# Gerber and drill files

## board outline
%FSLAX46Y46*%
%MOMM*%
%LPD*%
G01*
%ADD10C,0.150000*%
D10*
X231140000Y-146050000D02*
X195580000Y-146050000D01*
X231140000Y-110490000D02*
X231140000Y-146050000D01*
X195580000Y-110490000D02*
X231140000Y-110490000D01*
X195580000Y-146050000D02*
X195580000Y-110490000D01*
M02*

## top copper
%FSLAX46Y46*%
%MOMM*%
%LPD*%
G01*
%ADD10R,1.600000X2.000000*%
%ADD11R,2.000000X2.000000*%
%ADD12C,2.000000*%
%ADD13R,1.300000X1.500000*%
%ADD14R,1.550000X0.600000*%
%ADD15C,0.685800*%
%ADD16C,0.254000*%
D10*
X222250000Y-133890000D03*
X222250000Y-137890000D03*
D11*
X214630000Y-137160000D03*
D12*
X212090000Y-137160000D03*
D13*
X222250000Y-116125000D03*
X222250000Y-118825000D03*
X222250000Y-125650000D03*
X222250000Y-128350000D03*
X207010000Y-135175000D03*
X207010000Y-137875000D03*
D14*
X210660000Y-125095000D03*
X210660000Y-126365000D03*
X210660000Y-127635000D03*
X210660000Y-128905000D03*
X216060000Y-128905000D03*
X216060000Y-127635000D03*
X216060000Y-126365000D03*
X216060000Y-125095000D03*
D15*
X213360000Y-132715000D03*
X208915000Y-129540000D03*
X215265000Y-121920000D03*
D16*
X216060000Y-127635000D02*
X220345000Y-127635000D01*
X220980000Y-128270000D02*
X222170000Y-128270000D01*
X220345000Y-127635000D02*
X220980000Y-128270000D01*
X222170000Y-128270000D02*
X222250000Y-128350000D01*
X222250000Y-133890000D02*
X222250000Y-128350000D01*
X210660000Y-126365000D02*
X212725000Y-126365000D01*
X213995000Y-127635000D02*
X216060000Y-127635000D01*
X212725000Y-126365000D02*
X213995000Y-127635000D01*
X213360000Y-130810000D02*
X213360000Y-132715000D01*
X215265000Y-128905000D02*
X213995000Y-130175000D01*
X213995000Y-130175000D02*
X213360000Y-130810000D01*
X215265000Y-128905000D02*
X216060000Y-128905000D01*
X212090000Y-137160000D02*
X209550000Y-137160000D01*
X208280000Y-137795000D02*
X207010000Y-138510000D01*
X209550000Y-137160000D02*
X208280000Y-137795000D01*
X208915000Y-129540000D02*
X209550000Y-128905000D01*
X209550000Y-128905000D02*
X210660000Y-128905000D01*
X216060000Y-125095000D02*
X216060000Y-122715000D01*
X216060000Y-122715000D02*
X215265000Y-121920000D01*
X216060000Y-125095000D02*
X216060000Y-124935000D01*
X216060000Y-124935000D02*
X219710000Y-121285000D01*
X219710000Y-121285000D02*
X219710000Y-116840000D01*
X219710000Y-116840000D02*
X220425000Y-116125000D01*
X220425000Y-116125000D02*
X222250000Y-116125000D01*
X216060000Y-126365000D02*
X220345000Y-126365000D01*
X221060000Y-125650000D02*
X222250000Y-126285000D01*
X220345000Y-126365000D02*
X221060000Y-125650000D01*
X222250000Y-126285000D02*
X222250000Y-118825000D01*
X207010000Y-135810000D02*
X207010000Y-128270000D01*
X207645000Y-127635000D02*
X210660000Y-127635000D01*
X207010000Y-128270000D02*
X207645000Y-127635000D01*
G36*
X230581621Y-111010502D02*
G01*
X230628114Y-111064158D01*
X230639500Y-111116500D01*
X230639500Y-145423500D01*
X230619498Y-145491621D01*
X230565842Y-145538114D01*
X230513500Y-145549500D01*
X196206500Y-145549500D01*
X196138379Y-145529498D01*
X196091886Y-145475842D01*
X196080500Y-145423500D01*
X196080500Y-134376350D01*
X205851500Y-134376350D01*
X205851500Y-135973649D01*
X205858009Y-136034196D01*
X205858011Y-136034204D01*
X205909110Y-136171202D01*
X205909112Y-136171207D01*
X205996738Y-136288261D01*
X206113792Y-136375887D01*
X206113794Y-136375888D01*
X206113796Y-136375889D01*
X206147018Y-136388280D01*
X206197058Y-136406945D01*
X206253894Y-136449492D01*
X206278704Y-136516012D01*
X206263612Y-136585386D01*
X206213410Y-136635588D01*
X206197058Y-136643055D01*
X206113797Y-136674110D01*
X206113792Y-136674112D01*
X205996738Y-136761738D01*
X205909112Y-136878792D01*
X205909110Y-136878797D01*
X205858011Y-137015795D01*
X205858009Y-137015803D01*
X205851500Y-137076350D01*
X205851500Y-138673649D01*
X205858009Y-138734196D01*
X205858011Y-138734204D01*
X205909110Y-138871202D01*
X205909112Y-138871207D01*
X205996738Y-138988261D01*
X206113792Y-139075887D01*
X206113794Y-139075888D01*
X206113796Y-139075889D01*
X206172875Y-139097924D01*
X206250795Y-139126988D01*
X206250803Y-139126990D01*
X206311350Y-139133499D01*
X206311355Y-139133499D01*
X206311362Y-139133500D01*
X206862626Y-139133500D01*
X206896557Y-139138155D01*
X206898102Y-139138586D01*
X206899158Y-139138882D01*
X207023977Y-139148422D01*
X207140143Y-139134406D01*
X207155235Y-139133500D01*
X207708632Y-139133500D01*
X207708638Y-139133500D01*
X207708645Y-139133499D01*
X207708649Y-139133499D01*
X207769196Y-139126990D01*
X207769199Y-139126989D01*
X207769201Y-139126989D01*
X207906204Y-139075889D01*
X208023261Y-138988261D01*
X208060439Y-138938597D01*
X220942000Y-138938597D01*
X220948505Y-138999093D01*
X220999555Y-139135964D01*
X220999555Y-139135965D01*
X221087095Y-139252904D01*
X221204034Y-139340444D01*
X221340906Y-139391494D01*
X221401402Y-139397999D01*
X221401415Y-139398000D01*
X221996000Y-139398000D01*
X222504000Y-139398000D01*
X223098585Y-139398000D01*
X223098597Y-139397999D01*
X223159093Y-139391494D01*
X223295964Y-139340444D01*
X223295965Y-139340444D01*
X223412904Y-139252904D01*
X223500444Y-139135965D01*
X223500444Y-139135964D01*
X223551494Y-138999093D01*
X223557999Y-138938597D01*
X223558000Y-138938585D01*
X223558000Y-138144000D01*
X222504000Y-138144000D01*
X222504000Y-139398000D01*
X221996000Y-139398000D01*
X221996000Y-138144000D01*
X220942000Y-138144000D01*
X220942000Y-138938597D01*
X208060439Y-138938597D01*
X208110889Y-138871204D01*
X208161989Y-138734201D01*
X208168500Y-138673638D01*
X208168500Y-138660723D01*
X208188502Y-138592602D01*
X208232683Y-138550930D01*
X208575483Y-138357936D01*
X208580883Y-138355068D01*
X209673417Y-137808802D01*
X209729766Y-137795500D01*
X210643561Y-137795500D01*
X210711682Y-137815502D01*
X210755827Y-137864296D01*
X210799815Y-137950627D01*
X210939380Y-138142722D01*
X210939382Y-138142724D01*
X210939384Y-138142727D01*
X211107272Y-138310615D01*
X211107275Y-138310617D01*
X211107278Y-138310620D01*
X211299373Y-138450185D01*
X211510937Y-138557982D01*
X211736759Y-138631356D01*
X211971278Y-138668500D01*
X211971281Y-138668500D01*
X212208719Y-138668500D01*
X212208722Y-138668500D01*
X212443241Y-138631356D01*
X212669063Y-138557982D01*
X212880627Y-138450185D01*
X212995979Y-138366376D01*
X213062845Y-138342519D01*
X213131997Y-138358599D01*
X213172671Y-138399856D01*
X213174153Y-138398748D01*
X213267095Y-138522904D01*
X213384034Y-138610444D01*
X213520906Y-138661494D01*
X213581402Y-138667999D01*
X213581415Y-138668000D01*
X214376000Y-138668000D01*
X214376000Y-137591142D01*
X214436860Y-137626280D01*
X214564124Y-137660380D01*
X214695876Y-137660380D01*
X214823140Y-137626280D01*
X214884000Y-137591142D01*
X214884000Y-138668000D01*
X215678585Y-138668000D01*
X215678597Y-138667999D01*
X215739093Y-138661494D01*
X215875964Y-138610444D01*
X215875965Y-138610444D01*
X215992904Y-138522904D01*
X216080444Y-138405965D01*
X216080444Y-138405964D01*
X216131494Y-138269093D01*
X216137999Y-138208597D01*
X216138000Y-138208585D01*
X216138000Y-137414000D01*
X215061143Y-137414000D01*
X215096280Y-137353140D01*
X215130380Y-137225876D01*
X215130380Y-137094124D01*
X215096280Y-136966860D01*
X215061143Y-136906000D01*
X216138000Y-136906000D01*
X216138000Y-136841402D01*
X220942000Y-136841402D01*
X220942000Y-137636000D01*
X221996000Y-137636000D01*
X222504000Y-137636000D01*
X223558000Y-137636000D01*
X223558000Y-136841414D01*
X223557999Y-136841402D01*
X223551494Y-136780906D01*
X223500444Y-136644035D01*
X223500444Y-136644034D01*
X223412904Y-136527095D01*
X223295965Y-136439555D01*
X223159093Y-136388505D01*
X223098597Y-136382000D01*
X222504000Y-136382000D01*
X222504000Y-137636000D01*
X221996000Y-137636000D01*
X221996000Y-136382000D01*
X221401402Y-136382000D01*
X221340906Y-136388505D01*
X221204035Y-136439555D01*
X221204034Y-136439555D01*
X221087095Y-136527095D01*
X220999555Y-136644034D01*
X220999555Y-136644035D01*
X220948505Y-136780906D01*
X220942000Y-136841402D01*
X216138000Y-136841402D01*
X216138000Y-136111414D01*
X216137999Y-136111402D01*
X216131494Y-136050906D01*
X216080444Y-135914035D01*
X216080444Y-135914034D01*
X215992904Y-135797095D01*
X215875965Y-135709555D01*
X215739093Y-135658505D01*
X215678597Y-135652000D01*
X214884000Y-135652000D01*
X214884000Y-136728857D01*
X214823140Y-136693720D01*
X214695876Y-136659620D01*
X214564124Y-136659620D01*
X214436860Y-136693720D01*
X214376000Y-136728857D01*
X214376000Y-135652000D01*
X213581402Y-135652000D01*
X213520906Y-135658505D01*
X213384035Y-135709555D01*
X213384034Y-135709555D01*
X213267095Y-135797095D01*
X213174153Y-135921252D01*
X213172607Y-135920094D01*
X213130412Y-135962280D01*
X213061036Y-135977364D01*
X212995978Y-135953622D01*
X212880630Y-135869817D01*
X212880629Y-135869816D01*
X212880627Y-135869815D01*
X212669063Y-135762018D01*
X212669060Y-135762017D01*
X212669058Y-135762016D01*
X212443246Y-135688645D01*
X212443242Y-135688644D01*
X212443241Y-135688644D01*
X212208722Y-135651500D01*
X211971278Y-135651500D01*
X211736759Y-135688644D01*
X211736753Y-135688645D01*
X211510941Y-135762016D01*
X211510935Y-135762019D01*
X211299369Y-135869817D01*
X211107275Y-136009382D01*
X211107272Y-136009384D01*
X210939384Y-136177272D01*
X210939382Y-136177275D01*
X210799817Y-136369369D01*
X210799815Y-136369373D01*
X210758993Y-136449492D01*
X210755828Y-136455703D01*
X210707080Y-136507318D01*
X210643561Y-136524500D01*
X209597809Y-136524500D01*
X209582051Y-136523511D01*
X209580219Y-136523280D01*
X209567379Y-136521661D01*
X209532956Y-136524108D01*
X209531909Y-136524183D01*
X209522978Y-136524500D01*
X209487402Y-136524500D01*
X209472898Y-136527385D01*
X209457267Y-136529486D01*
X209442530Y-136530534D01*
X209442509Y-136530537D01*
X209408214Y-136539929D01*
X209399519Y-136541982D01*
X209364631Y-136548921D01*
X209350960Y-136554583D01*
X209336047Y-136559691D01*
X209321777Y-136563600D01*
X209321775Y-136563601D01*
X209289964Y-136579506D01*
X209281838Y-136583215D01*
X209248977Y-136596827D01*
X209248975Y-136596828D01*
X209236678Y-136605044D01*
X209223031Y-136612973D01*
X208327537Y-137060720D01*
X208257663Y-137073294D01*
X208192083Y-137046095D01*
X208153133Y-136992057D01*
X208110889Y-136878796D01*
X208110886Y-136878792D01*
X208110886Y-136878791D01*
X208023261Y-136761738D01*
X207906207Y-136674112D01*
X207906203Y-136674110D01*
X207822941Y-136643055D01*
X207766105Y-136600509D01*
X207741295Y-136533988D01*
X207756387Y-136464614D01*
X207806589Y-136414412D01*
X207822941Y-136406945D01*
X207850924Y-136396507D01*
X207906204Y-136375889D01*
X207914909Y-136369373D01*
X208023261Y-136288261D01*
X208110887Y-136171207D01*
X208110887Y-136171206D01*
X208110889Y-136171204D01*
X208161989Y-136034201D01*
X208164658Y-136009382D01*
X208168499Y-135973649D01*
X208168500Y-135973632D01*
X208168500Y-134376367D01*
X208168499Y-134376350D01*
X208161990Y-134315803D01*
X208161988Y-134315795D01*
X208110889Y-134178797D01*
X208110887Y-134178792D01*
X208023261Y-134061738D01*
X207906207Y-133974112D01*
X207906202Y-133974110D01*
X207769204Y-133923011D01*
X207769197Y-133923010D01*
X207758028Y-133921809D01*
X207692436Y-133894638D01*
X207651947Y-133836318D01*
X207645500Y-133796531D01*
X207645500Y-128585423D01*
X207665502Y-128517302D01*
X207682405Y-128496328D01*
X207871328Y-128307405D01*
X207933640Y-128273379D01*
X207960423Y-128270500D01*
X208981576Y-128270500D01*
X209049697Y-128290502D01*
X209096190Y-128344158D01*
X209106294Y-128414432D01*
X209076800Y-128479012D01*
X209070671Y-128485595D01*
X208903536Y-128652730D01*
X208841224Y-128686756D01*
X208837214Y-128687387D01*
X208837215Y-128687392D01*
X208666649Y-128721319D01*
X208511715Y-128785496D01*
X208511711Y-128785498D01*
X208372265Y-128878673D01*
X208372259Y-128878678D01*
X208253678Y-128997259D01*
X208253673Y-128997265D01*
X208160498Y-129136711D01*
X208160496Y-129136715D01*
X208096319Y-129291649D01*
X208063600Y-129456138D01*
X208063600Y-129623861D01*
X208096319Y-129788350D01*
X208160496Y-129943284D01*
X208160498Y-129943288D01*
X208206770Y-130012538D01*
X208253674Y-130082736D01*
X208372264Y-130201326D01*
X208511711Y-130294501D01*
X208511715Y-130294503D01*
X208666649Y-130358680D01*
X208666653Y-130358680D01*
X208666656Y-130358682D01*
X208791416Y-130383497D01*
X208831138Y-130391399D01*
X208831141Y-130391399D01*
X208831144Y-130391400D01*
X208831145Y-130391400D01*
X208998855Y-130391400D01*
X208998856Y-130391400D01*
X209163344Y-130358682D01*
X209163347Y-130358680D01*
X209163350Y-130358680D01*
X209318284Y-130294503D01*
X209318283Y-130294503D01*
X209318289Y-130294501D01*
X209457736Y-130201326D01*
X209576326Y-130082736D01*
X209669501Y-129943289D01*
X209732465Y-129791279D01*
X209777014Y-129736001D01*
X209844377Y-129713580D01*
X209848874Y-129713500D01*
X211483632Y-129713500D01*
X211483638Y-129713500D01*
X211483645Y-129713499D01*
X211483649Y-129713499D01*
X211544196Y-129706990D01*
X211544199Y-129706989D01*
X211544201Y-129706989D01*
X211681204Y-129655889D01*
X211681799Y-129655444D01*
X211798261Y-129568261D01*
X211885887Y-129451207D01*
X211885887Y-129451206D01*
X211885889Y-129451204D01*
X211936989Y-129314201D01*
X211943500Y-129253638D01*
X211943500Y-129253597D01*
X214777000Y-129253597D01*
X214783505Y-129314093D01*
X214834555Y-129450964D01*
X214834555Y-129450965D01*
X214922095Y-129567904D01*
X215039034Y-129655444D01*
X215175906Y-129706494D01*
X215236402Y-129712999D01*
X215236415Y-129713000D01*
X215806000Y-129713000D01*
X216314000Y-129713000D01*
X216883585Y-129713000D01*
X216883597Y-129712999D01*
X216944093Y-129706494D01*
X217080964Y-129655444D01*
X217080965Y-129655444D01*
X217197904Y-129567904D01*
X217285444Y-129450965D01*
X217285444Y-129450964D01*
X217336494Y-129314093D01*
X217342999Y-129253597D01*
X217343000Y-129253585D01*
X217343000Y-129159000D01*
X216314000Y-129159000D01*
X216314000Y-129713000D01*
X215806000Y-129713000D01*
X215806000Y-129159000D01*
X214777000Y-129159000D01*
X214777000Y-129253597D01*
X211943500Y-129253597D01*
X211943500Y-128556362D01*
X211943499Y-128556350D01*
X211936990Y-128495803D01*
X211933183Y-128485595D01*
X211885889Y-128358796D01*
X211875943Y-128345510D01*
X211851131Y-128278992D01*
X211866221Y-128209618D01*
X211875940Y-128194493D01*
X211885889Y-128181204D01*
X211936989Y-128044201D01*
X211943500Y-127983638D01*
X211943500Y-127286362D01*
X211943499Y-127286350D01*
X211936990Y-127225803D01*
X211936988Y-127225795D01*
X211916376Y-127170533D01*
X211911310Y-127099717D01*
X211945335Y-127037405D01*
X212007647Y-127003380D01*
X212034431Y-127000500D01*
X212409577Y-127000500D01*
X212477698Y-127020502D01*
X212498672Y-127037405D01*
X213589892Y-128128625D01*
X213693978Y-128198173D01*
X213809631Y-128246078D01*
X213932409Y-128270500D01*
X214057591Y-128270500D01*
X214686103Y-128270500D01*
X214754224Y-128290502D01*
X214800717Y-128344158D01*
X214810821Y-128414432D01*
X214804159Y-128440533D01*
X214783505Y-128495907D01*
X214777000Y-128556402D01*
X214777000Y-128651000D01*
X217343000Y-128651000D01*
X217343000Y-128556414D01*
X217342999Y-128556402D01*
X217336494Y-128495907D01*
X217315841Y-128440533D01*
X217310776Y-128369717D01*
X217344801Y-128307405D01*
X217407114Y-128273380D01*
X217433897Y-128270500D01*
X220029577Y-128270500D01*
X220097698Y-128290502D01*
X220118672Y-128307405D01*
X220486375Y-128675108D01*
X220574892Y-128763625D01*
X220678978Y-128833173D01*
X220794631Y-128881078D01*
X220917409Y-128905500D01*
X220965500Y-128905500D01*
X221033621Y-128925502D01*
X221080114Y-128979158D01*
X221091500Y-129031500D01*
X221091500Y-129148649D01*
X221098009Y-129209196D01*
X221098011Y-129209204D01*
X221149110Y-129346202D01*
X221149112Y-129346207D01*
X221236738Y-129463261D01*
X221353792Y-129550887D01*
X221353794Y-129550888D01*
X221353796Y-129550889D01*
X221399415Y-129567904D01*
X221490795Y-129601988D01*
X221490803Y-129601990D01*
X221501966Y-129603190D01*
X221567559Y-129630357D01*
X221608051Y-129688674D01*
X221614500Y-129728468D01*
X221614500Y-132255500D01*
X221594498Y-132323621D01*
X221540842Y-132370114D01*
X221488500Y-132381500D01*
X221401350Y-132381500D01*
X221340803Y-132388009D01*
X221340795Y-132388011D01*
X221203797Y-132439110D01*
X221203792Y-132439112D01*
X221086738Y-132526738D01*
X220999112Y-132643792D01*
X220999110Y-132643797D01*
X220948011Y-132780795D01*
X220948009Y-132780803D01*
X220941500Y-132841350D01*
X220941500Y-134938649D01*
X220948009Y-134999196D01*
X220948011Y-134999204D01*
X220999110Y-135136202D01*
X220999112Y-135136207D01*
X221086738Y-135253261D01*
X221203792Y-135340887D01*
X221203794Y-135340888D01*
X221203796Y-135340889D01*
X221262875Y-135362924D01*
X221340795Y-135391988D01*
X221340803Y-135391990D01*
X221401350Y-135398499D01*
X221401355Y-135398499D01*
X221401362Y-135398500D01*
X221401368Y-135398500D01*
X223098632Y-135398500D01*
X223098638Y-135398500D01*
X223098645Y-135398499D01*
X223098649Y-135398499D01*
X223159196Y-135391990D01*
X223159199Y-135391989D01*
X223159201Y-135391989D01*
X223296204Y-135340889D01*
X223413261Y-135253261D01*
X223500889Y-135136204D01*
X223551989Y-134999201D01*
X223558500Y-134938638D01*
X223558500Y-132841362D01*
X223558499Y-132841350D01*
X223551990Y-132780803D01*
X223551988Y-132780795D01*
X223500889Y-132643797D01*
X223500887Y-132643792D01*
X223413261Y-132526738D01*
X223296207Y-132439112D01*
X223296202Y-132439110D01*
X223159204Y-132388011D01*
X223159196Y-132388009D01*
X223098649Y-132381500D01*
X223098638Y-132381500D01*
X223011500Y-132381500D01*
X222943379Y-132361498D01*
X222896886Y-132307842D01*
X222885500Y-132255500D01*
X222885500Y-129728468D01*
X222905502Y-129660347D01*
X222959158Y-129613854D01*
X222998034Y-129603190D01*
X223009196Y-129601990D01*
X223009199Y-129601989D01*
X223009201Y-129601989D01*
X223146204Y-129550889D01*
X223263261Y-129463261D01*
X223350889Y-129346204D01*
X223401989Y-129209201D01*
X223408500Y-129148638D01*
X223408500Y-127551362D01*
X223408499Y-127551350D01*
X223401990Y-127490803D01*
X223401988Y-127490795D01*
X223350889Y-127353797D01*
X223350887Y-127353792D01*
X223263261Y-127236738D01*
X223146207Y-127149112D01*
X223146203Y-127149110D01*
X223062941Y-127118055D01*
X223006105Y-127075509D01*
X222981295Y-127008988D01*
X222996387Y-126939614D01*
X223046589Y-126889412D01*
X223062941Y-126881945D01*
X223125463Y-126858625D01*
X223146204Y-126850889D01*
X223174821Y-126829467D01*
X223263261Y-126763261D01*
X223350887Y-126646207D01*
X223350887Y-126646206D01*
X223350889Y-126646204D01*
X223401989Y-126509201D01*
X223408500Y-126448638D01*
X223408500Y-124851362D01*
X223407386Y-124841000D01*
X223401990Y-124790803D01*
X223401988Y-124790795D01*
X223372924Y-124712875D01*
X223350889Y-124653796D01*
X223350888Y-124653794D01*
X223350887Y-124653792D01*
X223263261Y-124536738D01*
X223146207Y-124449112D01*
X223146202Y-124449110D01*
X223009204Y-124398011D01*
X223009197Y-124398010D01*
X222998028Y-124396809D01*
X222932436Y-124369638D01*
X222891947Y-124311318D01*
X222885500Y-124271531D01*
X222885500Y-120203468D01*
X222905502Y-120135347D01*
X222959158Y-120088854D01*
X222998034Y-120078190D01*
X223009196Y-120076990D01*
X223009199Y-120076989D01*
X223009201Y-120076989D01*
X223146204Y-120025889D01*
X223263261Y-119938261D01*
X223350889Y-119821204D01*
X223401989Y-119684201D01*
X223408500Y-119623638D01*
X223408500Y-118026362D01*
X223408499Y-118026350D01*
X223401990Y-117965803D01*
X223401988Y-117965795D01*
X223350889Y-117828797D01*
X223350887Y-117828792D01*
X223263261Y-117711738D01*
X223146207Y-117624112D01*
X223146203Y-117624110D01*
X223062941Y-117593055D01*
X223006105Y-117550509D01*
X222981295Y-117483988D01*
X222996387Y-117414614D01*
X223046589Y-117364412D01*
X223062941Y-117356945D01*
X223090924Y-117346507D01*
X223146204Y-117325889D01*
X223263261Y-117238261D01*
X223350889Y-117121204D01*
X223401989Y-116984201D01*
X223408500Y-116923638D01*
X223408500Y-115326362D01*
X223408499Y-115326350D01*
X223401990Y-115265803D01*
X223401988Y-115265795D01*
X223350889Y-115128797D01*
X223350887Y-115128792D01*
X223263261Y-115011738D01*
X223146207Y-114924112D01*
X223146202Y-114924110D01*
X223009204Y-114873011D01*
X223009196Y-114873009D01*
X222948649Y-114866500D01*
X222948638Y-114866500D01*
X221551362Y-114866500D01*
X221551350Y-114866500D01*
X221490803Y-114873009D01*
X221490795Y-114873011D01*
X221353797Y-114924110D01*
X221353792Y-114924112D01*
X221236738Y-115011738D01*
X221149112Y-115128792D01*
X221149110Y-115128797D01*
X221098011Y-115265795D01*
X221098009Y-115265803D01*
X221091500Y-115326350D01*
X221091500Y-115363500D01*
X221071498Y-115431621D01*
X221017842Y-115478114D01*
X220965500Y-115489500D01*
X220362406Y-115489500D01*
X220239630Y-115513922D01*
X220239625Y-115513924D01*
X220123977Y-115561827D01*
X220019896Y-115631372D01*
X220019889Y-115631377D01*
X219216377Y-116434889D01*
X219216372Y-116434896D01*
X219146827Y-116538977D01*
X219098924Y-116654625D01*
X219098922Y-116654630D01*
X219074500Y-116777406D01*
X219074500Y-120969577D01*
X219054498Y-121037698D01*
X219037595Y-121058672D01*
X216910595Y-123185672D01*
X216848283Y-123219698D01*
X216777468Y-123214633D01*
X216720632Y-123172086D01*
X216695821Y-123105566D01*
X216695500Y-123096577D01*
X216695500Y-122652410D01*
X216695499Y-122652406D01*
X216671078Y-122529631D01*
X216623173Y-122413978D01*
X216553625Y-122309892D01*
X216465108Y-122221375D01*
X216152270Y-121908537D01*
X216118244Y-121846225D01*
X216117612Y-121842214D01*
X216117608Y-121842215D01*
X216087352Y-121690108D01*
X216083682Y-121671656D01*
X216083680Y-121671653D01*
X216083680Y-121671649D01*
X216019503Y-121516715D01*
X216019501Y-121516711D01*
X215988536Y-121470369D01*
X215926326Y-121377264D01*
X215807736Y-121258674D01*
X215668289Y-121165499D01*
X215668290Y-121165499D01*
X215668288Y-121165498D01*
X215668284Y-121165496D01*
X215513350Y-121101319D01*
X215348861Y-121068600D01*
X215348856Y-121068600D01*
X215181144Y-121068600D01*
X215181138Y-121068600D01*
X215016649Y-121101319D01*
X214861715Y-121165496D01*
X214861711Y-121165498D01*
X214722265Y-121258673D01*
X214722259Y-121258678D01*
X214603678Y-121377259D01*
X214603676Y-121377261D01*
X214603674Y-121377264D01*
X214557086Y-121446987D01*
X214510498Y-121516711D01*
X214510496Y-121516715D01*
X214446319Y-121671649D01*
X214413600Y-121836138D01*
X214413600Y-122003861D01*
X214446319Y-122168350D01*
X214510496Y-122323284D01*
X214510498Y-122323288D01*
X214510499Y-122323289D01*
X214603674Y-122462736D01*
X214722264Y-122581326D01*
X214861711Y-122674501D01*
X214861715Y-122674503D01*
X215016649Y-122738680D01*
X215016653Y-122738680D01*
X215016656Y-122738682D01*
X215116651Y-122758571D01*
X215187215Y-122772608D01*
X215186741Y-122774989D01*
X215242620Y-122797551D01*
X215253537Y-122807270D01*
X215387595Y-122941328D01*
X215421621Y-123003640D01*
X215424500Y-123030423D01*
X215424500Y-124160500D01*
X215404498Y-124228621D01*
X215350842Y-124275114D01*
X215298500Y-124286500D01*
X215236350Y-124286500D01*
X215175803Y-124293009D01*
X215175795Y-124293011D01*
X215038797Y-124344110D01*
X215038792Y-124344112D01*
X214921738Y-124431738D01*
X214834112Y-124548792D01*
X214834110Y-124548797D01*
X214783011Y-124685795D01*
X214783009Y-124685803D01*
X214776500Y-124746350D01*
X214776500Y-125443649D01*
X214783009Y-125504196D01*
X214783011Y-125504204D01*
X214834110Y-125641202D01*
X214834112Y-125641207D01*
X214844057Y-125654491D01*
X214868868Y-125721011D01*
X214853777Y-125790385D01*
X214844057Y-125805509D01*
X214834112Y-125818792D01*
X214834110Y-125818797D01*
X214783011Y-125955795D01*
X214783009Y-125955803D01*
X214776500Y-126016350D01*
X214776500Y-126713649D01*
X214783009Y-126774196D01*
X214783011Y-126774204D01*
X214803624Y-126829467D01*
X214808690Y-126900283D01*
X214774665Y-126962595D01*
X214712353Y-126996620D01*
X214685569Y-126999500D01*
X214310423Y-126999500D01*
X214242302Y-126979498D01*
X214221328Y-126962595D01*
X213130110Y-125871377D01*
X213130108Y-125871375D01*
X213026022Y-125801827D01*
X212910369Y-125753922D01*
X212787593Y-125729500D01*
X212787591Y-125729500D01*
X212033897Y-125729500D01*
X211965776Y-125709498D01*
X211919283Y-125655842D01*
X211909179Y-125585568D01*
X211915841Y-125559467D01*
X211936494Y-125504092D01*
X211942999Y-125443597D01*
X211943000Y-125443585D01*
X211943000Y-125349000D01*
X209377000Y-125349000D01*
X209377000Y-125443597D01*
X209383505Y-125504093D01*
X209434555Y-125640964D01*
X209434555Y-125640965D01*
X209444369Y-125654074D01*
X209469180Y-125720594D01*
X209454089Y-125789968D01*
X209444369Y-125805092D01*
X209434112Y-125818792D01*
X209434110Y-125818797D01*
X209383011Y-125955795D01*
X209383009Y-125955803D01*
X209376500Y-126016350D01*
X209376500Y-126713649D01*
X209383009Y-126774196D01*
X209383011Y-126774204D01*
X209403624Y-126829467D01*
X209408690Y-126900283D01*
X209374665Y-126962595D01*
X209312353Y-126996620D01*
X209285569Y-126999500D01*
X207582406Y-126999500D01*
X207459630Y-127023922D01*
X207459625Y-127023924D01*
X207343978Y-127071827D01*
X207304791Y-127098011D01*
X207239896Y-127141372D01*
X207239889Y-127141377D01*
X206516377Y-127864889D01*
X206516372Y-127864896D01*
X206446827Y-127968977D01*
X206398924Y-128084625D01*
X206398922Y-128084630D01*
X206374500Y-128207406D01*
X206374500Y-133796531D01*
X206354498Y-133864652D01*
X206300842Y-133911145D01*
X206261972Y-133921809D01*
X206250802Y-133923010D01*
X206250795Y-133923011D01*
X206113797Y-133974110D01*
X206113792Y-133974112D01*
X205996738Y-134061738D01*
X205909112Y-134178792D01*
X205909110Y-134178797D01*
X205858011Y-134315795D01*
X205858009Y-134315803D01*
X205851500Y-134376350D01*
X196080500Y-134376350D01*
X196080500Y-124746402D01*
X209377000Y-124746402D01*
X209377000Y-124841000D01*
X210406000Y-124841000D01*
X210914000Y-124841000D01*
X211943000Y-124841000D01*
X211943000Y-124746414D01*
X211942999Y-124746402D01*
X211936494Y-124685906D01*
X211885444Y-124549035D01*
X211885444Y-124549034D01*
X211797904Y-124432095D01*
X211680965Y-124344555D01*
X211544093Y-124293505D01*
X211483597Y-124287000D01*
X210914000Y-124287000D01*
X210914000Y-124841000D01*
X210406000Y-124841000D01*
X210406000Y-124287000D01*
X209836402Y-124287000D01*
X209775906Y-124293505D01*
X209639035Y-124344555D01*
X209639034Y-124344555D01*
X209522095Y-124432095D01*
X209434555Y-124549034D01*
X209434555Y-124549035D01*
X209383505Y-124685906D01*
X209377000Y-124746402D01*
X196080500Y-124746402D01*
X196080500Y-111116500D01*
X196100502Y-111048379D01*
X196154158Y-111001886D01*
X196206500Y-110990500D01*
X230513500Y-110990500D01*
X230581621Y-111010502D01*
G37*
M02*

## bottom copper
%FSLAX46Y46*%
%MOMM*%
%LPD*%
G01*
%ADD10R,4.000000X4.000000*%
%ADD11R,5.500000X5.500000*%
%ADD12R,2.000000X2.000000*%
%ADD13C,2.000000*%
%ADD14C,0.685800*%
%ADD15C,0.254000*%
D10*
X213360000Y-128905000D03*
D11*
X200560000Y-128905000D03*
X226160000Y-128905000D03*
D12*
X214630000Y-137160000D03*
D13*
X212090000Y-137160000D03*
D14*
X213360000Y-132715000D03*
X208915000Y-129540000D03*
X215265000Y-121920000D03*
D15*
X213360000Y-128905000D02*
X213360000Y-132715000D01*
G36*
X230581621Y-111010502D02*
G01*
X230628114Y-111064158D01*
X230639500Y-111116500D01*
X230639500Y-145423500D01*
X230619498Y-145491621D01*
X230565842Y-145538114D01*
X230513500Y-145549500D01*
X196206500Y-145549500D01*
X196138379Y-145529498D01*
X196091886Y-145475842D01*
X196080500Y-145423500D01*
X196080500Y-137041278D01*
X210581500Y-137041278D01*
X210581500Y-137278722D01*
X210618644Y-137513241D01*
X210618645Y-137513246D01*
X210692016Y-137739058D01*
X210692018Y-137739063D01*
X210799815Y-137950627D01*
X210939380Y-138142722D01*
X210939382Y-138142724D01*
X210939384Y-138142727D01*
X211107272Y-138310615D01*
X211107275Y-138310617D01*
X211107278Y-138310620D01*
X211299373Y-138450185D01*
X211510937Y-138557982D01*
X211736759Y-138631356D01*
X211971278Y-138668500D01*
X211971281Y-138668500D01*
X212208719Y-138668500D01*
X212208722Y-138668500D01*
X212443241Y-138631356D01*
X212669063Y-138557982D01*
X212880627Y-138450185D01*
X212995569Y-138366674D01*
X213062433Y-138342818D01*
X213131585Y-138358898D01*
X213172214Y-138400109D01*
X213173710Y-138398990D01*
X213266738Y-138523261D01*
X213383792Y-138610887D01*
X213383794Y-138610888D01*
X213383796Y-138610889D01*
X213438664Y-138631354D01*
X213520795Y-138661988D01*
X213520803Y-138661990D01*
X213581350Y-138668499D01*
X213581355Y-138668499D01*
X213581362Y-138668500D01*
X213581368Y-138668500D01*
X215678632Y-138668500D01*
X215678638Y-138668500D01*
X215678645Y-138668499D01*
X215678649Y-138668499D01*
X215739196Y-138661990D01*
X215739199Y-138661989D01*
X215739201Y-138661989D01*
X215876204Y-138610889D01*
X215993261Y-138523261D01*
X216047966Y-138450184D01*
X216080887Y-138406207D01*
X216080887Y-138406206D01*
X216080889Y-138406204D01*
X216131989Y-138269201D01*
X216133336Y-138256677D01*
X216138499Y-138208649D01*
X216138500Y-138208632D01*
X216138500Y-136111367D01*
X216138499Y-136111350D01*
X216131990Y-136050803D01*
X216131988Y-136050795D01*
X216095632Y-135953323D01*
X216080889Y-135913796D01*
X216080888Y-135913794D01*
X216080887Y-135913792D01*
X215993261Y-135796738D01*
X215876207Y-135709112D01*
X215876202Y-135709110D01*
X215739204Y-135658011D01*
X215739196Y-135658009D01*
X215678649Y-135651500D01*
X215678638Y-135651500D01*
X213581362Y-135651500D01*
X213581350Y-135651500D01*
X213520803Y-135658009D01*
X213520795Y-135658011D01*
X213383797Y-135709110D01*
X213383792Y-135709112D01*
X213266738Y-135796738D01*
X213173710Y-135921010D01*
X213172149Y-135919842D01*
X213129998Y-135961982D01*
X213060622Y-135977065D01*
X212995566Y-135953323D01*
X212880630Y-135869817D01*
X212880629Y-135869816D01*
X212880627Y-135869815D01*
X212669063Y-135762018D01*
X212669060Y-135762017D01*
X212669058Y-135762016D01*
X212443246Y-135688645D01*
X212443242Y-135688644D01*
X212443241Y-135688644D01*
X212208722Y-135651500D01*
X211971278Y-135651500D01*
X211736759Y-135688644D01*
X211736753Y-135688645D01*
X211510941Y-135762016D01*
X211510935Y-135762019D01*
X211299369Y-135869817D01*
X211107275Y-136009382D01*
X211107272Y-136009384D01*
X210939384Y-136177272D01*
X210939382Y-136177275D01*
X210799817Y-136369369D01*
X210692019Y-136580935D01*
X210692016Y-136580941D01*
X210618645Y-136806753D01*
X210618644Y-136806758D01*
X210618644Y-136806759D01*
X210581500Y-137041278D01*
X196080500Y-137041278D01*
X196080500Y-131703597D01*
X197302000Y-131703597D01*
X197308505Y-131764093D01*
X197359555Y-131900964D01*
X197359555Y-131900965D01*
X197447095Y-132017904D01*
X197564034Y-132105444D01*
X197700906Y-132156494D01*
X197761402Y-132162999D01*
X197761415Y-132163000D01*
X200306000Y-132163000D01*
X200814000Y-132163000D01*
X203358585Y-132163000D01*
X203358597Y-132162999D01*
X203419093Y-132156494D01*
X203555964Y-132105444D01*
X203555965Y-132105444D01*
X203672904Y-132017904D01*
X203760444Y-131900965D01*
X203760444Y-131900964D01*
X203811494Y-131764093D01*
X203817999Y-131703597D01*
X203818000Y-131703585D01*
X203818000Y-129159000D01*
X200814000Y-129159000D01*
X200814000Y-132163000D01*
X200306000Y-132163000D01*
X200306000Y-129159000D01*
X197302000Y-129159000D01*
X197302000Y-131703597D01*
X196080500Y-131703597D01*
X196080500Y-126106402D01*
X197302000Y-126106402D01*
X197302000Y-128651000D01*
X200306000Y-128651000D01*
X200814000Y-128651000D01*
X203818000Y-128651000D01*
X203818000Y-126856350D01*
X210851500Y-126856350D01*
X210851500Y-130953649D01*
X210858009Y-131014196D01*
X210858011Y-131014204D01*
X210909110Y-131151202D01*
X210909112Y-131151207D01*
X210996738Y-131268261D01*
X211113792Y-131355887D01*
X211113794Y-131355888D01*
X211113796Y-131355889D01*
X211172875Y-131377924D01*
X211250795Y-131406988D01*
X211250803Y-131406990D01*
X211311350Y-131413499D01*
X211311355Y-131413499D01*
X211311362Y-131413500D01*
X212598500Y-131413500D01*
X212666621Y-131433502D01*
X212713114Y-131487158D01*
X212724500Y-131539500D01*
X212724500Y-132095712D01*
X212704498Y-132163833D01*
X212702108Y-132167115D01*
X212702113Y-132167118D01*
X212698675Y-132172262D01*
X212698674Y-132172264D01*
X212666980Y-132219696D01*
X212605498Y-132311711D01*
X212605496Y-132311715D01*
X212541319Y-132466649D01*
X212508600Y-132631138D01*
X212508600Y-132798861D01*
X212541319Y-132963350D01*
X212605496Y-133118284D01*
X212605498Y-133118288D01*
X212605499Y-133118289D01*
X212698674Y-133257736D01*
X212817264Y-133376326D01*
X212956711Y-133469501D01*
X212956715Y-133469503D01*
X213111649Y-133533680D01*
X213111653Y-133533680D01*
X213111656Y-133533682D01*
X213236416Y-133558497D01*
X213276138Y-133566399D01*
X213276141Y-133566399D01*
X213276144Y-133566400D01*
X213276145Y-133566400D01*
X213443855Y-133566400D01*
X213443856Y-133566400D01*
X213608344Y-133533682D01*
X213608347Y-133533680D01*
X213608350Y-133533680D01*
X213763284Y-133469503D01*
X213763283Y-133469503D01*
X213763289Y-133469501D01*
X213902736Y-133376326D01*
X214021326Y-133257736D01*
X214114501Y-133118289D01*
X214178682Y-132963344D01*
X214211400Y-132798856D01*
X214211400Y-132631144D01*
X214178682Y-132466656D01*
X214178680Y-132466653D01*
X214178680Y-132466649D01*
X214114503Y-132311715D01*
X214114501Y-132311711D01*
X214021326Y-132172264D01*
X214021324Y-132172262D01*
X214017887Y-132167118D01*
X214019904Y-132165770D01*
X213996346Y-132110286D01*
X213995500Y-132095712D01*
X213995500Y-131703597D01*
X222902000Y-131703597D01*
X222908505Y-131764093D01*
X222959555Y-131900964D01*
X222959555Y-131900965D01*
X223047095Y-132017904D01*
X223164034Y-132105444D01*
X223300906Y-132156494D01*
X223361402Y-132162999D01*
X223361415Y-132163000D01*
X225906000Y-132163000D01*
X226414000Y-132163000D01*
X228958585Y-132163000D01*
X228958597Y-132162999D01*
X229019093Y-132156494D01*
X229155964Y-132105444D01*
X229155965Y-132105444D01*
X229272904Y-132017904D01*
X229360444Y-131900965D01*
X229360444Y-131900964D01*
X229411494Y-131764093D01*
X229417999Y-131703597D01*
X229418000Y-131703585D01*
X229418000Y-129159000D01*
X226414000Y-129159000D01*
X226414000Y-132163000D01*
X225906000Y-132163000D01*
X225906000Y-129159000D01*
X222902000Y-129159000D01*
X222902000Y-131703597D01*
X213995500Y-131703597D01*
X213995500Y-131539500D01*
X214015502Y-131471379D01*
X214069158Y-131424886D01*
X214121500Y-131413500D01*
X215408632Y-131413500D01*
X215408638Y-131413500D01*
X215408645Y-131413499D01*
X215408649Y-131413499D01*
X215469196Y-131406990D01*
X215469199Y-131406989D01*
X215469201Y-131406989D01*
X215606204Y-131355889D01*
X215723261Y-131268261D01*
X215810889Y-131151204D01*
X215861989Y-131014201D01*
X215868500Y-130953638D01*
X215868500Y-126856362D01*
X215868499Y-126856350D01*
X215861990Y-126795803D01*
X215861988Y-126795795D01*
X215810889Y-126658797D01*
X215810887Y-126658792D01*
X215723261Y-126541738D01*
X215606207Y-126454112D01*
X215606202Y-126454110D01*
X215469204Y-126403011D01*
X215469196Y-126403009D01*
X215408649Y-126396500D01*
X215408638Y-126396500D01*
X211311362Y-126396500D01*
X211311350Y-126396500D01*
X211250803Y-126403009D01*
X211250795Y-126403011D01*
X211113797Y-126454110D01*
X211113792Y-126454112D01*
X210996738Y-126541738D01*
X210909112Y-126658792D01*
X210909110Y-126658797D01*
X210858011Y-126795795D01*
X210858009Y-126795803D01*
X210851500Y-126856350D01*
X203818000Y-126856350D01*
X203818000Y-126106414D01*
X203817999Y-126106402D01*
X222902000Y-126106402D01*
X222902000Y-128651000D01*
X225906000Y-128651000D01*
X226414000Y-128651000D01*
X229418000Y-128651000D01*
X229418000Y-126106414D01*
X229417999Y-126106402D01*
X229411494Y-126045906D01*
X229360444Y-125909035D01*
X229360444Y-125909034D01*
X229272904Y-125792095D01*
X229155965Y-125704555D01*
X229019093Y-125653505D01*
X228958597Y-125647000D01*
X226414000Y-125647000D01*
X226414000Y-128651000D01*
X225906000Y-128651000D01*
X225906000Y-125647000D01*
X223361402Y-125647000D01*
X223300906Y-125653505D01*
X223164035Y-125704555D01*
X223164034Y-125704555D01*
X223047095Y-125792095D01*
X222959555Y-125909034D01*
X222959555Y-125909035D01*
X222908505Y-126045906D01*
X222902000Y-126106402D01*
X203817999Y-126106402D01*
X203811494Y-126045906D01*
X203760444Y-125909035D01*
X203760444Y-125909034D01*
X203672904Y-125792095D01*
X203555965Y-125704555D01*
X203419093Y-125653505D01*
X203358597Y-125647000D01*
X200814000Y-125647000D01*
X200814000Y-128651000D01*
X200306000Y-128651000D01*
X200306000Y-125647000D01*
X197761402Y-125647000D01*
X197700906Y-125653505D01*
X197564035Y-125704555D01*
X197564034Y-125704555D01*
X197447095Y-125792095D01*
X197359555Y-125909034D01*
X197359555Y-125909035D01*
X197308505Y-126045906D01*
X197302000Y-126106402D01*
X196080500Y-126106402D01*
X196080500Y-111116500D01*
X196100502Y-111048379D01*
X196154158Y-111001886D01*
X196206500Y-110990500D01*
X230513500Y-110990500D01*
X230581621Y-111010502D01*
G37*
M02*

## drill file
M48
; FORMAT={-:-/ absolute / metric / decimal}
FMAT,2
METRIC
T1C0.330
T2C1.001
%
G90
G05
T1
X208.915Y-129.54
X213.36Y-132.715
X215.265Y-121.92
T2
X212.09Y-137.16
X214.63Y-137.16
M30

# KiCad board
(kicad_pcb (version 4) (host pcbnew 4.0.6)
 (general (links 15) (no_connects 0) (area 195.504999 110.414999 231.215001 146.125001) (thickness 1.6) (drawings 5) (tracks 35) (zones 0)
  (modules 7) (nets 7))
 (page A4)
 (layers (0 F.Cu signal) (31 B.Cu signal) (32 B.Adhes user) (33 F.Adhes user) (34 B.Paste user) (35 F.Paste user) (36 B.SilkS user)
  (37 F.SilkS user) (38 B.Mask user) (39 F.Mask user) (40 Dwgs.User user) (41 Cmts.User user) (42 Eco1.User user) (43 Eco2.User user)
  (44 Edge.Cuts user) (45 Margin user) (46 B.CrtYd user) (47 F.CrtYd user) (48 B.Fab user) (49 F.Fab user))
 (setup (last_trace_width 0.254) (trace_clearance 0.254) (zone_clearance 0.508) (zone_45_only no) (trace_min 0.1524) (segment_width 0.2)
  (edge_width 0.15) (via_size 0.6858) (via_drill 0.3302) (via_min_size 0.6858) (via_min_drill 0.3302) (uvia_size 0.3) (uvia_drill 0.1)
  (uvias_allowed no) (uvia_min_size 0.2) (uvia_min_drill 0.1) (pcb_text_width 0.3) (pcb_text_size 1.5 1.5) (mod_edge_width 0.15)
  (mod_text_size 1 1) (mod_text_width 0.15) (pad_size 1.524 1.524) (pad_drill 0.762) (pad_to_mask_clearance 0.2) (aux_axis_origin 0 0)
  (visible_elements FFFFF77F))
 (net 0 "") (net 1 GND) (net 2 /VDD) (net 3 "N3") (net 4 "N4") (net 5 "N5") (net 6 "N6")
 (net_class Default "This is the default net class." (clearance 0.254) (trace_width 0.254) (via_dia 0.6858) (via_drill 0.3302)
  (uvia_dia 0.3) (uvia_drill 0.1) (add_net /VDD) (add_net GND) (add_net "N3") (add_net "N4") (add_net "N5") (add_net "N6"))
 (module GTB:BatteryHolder (layer B.Cu) (at 213.36 128.905)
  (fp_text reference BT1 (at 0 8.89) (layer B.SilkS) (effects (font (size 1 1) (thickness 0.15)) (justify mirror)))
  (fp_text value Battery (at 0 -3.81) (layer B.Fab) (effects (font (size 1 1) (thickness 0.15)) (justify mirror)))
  (pad 2 smd rect (at 0 0) (size 4 4) (layers B.Cu B.Paste B.Mask) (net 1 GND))
  (pad 1 smd rect (at -12.8 0) (size 5.5 5.5) (layers B.Cu B.Paste B.Mask) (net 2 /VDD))
  (pad 1 smd rect (at 12.8 0) (size 5.5 5.5) (layers B.Cu B.Paste B.Mask) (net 2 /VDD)))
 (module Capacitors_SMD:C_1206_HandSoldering (layer F.Cu) (at 222.25 135.89 270)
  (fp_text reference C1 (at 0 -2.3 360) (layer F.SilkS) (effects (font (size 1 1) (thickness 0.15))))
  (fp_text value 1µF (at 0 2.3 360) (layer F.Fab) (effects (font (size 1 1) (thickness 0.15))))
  (pad 1 smd rect (at -2 0 270) (size 2 1.6) (layers F.Cu F.Paste F.Mask) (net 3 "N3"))
  (pad 2 smd rect (at 2 0 270) (size 2 1.6) (layers F.Cu F.Paste F.Mask) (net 1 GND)))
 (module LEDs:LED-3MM (layer F.Cu) (at 214.63 137.16 180)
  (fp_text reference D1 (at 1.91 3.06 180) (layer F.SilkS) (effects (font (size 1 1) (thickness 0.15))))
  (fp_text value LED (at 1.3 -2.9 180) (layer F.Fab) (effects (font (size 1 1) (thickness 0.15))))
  (pad 1 thru_hole rect (at 0 0 270) (size 2 2) (drill 1.00076) (layers *.Cu *.Mask) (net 1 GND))
  (pad 2 thru_hole circle (at 2.54 0 180) (size 2 2) (drill 1.00076) (layers *.Cu *.Mask) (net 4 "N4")))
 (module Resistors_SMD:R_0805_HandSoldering (layer F.Cu) (at 222.25 117.475 270)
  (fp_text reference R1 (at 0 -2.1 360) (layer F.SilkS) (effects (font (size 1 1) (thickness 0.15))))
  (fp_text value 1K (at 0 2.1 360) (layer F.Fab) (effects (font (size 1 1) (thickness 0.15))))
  (pad 1 smd rect (at -1.35 0 270) (size 1.5 1.3) (layers F.Cu F.Paste F.Mask) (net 2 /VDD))
  (pad 2 smd rect (at 1.35 0 270) (size 1.5 1.3) (layers F.Cu F.Paste F.Mask) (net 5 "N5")))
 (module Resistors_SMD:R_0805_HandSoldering (layer F.Cu) (at 222.25 127 270)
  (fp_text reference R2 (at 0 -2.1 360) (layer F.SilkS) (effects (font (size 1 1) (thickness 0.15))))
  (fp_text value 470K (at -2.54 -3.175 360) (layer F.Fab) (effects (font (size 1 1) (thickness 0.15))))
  (pad 1 smd rect (at -1.35 0 270) (size 1.5 1.3) (layers F.Cu F.Paste F.Mask) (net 5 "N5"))
  (pad 2 smd rect (at 1.35 0 270) (size 1.5 1.3) (layers F.Cu F.Paste F.Mask) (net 3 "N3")))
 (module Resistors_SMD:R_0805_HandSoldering (layer F.Cu) (at 207.01 136.525 270)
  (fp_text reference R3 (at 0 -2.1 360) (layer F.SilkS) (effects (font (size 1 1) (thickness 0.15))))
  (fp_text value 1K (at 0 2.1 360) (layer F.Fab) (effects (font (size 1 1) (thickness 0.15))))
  (pad 1 smd rect (at -1.35 0 270) (size 1.5 1.3) (layers F.Cu F.Paste F.Mask) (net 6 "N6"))
  (pad 2 smd rect (at 1.35 0 270) (size 1.5 1.3) (layers F.Cu F.Paste F.Mask) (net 4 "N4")))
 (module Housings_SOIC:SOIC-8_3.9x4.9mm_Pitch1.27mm (layer F.Cu) (at 213.36 127)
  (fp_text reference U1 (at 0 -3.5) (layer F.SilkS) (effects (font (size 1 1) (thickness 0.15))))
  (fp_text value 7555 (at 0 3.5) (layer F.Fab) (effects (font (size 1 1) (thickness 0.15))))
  (pad 1 smd rect (at -2.7 -1.905) (size 1.55 0.6) (layers F.Cu F.Paste F.Mask) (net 1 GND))
  (pad 2 smd rect (at -2.7 -0.635) (size 1.55 0.6) (layers F.Cu F.Paste F.Mask) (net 3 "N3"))
  (pad 3 smd rect (at -2.7 0.635) (size 1.55 0.6) (layers F.Cu F.Paste F.Mask) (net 6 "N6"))
  (pad 4 smd rect (at -2.7 1.905) (size 1.55 0.6) (layers F.Cu F.Paste F.Mask) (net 2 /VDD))
  (pad 5 smd rect (at 2.7 1.905) (size 1.55 0.6) (layers F.Cu F.Paste F.Mask) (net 1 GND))
  (pad 6 smd rect (at 2.7 0.635) (size 1.55 0.6) (layers F.Cu F.Paste F.Mask) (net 3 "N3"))
  (pad 7 smd rect (at 2.7 -0.635) (size 1.55 0.6) (layers F.Cu F.Paste F.Mask) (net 5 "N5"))
  (pad 8 smd rect (at 2.7 -1.905) (size 1.55 0.6) (layers F.Cu F.Paste F.Mask) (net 2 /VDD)))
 (gr_line (start 231.14 146.05) (end 195.58 146.05) (angle 90) (layer Edge.Cuts) (width 0.15))
 (gr_line (start 231.14 110.49) (end 231.14 146.05) (angle 90) (layer Edge.Cuts) (width 0.15))
 (gr_line (start 195.58 110.49) (end 231.14 110.49) (angle 90) (layer Edge.Cuts) (width 0.15))
 (gr_line (start 195.58 146.05) (end 195.58 110.49) (angle 90) (layer Edge.Cuts) (width 0.15))
 (segment (start 216.06 127.635) (end 220.345 127.635) (width 0.254) (layer F.Cu) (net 3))
 (segment (start 220.98 128.27) (end 222.17 128.27) (width 0.254) (layer F.Cu) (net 3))
 (segment (start 220.345 127.635) (end 220.98 128.27) (width 0.254) (layer F.Cu) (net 3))
 (segment (start 222.17 128.27) (end 222.25 128.35) (width 0.254) (layer F.Cu) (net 3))
 (segment (start 222.25 133.89) (end 222.25 128.35) (width 0.254) (layer F.Cu) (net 3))
 (segment (start 210.66 126.365) (end 212.725 126.365) (width 0.254) (layer F.Cu) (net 3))
 (segment (start 213.995 127.635) (end 216.06 127.635) (width 0.254) (layer F.Cu) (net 3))
 (segment (start 212.725 126.365) (end 213.995 127.635) (width 0.254) (layer F.Cu) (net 3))
 (segment (start 213.36 128.905) (end 213.36 132.715) (width 0.254) (layer B.Cu) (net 1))
 (via (at 213.36 132.715) (size 0.6858) (drill 0.3302) (layers F.Cu B.Cu) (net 1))
 (segment (start 213.36 130.81) (end 213.36 132.715) (width 0.254) (layer F.Cu) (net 1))
 (segment (start 215.265 128.905) (end 213.995 130.175) (width 0.254) (layer F.Cu) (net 1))
 (segment (start 213.995 130.175) (end 213.36 130.81) (width 0.254) (layer F.Cu) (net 1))
 (segment (start 215.265 128.905) (end 216.06 128.905) (width 0.254) (layer F.Cu) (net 1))
 (segment (start 212.09 137.16) (end 209.55 137.16) (width 0.254) (layer F.Cu) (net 4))
 (segment (start 208.28 137.795) (end 207.01 138.51) (width 0.254) (layer F.Cu) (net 4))
 (segment (start 209.55 137.16) (end 208.28 137.795) (width 0.254) (layer F.Cu) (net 4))
 (via (at 208.915 129.54) (size 0.6858) (drill 0.3302) (layers F.Cu B.Cu) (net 2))
 (segment (start 208.915 129.54) (end 209.55 128.905) (width 0.254) (layer F.Cu) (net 2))
 (segment (start 209.55 128.905) (end 210.66 128.905) (width 0.254) (layer F.Cu) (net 2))
 (via (at 215.265 121.92) (size 0.6858) (drill 0.3302) (layers F.Cu B.Cu) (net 2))
 (segment (start 216.06 125.095) (end 216.06 122.715) (width 0.254) (layer F.Cu) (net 2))
 (segment (start 216.06 122.715) (end 215.265 121.92) (width 0.254) (layer F.Cu) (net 2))
 (segment (start 216.06 125.095) (end 216.06 124.935) (width 0.254) (layer F.Cu) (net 2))
 (segment (start 216.06 124.935) (end 219.71 121.285) (width 0.254) (layer F.Cu) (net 2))
 (segment (start 219.71 121.285) (end 219.71 116.84) (width 0.254) (layer F.Cu) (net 2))
 (segment (start 219.71 116.84) (end 220.425 116.125) (width 0.254) (layer F.Cu) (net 2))
 (segment (start 220.425 116.125) (end 222.25 116.125) (width 0.254) (layer F.Cu) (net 2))
 (segment (start 216.06 126.365) (end 220.345 126.365) (width 0.254) (layer F.Cu) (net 5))
 (segment (start 221.06 125.65) (end 222.25 126.285) (width 0.254) (layer F.Cu) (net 5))
 (segment (start 220.345 126.365) (end 221.06 125.65) (width 0.254) (layer F.Cu) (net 5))
 (segment (start 222.25 126.285) (end 222.25 118.825) (width 0.254) (layer F.Cu) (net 5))
 (segment (start 207.01 135.81) (end 207.01 128.27) (width 0.254) (layer F.Cu) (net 6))
 (segment (start 207.645 127.635) (end 210.66 127.635) (width 0.254) (layer F.Cu) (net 6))
 (segment (start 207.01 128.27) (end 207.645 127.635) (width 0.254) (layer F.Cu) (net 6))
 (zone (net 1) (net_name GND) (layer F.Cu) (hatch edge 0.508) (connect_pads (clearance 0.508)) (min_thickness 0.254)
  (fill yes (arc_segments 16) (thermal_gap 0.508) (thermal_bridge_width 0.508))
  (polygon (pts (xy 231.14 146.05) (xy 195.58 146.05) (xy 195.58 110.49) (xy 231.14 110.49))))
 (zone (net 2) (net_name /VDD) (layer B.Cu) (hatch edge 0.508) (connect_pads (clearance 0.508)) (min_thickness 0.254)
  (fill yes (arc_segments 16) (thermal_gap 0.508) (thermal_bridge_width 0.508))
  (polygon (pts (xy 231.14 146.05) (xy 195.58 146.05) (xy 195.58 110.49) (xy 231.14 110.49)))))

